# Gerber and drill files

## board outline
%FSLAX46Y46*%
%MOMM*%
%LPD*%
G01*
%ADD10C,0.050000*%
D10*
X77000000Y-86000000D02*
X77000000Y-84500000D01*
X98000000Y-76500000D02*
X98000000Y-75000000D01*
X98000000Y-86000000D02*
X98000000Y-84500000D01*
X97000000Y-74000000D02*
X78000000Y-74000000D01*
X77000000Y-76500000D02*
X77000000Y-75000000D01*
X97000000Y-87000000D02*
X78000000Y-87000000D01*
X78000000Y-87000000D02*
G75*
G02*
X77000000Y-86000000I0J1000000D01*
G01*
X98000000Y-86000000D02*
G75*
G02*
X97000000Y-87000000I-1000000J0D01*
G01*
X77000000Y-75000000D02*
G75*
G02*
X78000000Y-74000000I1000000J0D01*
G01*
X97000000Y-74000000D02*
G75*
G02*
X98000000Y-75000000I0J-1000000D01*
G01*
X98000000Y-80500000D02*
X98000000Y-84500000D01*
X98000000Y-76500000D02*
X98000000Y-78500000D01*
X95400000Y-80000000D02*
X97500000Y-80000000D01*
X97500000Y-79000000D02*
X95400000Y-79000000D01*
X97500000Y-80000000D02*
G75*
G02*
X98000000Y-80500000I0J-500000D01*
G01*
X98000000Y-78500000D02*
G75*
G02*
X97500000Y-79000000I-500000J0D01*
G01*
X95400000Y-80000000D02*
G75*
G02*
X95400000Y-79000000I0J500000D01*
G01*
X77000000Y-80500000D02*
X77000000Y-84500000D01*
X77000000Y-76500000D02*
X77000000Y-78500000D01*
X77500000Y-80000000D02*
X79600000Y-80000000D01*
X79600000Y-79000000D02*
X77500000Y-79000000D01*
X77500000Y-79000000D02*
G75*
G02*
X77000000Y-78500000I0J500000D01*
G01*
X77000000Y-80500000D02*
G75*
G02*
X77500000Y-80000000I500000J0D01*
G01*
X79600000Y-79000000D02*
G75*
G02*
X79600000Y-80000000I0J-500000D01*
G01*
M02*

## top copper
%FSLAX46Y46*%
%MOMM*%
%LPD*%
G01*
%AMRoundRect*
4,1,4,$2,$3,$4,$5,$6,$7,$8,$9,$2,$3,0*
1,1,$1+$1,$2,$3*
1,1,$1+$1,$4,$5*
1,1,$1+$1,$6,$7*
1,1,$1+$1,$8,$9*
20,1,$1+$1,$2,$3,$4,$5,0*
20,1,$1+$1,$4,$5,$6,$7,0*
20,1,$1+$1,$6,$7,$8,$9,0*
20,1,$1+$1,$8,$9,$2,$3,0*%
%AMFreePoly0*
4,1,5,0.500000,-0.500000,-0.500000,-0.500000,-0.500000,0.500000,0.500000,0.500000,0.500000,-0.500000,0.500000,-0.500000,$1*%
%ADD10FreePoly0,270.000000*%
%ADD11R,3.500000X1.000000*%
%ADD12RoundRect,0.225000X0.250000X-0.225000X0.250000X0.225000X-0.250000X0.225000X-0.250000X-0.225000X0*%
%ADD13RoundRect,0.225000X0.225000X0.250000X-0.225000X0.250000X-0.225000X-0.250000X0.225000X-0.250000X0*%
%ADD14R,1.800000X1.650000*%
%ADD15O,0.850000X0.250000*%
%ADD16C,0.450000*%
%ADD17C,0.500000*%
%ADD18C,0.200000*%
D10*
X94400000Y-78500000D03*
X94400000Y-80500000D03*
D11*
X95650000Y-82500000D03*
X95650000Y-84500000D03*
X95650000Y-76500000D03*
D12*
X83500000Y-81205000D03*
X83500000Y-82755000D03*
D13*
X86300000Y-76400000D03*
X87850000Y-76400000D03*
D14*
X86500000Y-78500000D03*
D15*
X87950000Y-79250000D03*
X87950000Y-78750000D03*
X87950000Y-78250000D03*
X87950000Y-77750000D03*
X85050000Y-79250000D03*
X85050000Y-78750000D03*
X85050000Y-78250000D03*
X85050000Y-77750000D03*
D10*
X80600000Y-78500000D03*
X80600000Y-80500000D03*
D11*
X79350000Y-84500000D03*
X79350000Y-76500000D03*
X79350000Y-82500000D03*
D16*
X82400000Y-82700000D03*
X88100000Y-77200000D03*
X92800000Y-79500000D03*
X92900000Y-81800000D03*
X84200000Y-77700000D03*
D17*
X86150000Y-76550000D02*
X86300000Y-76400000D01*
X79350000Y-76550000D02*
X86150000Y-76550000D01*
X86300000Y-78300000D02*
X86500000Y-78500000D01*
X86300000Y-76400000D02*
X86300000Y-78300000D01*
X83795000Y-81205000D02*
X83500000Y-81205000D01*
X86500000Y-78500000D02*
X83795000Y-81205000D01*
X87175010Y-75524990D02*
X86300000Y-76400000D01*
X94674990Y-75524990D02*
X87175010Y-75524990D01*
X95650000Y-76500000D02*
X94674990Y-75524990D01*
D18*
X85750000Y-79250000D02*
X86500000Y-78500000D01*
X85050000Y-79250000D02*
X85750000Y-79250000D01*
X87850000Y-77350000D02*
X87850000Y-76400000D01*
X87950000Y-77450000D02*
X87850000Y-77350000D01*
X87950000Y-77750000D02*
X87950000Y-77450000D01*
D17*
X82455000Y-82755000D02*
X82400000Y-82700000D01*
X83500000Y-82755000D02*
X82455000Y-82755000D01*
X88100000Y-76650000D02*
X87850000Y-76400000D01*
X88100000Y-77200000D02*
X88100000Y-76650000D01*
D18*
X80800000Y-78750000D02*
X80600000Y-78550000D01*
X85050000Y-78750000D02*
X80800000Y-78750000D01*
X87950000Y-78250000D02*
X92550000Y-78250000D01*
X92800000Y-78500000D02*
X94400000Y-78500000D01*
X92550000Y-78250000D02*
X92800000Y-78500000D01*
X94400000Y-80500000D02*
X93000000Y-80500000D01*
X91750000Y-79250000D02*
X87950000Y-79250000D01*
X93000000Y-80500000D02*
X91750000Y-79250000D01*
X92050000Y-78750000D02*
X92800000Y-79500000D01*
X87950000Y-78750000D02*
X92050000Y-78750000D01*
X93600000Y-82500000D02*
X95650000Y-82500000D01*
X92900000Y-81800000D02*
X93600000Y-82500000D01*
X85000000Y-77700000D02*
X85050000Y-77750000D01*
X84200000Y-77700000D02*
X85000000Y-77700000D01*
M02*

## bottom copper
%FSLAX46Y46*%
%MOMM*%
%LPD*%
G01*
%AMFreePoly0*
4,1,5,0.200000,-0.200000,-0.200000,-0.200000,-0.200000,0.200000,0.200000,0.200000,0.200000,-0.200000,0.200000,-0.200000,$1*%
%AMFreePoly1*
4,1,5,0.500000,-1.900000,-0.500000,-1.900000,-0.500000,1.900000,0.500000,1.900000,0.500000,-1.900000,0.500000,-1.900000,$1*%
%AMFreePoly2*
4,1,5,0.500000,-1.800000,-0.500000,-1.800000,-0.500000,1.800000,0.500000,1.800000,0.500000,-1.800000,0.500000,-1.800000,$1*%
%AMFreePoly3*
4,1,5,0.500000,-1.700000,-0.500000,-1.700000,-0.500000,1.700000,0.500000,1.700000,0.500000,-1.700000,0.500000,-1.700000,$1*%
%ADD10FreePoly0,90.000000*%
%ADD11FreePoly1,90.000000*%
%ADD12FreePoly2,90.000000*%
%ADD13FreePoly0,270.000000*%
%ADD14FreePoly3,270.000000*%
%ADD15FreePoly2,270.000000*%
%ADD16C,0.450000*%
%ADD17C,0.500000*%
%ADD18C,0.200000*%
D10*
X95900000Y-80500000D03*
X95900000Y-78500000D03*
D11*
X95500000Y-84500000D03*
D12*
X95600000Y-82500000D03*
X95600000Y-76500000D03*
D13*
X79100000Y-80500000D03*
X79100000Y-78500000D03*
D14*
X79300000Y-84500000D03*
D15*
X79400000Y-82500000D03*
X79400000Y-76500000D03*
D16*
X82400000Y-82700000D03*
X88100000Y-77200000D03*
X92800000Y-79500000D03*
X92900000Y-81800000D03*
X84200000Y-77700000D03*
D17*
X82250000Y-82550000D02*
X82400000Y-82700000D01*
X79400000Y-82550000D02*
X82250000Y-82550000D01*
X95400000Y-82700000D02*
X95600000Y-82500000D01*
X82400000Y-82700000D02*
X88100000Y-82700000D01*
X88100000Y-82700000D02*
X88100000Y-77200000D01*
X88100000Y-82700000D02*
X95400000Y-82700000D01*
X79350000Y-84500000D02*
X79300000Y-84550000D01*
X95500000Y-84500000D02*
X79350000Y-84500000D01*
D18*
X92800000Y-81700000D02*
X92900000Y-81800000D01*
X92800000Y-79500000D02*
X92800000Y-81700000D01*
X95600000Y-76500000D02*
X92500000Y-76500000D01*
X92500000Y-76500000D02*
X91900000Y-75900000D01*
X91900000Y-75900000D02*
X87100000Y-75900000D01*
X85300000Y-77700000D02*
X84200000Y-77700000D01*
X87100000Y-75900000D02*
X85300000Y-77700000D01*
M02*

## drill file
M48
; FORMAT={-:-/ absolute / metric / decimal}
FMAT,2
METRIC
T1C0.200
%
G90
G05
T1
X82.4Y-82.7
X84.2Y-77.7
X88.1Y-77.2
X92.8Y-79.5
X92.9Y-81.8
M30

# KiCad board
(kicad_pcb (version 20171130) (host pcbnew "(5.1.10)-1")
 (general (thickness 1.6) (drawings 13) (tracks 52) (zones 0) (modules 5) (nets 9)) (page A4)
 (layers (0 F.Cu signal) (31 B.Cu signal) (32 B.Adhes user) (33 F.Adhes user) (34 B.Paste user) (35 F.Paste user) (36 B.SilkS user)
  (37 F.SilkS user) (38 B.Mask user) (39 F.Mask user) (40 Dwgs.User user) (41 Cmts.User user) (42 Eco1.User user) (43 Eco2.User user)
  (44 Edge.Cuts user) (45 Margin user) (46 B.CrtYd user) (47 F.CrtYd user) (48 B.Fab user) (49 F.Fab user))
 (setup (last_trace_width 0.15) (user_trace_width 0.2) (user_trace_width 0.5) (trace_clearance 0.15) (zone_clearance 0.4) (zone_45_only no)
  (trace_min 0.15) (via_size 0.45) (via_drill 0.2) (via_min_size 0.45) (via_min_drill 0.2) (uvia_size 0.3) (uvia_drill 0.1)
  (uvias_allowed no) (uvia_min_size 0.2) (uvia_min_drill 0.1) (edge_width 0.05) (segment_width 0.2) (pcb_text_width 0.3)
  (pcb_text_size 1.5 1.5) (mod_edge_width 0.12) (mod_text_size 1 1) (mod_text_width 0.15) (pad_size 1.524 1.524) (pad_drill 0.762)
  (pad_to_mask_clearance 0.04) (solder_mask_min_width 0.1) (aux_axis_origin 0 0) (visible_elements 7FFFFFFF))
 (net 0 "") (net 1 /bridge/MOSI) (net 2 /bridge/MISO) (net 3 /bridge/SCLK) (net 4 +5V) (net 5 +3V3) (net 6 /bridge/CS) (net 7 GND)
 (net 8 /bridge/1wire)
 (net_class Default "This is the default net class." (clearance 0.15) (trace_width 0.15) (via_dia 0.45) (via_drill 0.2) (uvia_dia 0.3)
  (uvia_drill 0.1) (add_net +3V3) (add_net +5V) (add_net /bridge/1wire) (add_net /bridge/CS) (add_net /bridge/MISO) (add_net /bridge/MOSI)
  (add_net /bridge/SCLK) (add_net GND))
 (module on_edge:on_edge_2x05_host (layer F.Cu) (at 98 80.5 270)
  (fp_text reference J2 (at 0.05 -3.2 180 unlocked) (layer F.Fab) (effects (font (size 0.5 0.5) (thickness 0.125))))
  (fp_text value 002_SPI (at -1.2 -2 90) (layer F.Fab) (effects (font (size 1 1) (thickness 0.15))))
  (fp_line (start 0 0) (end 4 0) (layer Edge.Cuts) (width 0.05))
  (fp_line (start -4 0) (end -2 0) (layer Edge.Cuts) (width 0.05))
  (fp_line (start -0.5 2.6) (end -0.5 0.5) (layer Edge.Cuts) (width 0.05))
  (fp_line (start -1.5 0.5) (end -1.5 2.6) (layer Edge.Cuts) (width 0.05))
  (fp_arc (start 0 0.5) (end 0 0) (angle -90) (layer Edge.Cuts) (width 0.05))
  (fp_arc (start -2 0.5) (end -1.5 0.5) (angle -90) (layer Edge.Cuts) (width 0.05))
  (fp_arc (start -1 2.6) (end -1.5 2.6) (angle -180) (layer Edge.Cuts) (width 0.05))
  (pad 2 smd custom (at -2 3.6 270) (size 1 1) (layers F.Cu F.Mask) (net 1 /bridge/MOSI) (zone_connect 0)
   (options (clearance outline) (anchor rect)) (primitives))
  (pad 3 smd custom (at 0 3.6 270) (size 1 1) (layers F.Cu F.Mask) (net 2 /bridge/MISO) (zone_connect 0)
   (options (clearance outline) (anchor rect)) (primitives))
  (pad 8 smd custom (at 0 2.1 90) (size 0.4 0.4) (layers B.Cu B.Mask) (zone_connect 0) (options (clearance outline) (anchor rect))
   (primitives))
  (pad 7 smd custom (at -2 2.1 90) (size 0.4 0.4) (layers B.Cu B.Mask) (zone_connect 0) (options (clearance outline) (anchor rect))
   (primitives))
  (pad 4 smd rect (at 2 2.35 270) (size 1 3.5) (layers F.Cu F.Mask) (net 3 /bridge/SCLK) (zone_connect 0))
  (pad 10 smd custom (at 4 2.5 90) (size 1 3.8) (layers B.Cu B.Mask) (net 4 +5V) (zone_connect 0)
   (options (clearance outline) (anchor rect)) (primitives))
  (pad 9 smd custom (at 2 2.4 90) (size 1 3.6) (layers B.Cu B.Mask) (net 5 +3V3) (zone_connect 0)
   (options (clearance outline) (anchor rect)) (primitives))
  (pad 6 smd custom (at -4 2.4 90) (size 1 3.6) (layers B.Cu B.Mask) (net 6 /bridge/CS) (zone_connect 0)
   (options (clearance outline) (anchor rect)) (primitives))
  (pad 5 smd rect (at 4 2.35 270) (size 1 3.5) (layers F.Cu F.Mask) (zone_connect 0))
  (pad 1 smd rect (at -4 2.35 270) (size 1 3.5) (layers F.Cu F.Mask) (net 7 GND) (zone_connect 0)))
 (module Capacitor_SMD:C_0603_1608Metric (layer F.Cu) (at 83.5 81.98 90)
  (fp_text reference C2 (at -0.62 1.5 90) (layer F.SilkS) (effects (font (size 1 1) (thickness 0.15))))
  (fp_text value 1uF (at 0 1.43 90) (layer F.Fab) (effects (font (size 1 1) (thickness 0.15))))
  (pad 2 smd roundrect (at 0.775 0 90) (size 0.9 0.95) (layers F.Cu F.Paste F.Mask) (roundrect_rratio 0.25) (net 7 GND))
  (pad 1 smd roundrect (at -0.775 0 90) (size 0.9 0.95) (layers F.Cu F.Paste F.Mask) (roundrect_rratio 0.25) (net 5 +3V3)))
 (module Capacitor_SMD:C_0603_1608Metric (layer F.Cu) (at 87.075 76.4 180)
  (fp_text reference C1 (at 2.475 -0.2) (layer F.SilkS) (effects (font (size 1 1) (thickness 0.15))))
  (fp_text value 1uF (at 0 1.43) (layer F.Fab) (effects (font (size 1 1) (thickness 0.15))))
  (pad 2 smd roundrect (at 0.775 0 180) (size 0.9 0.95) (layers F.Cu F.Paste F.Mask) (roundrect_rratio 0.25) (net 7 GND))
  (pad 1 smd roundrect (at -0.775 0 180) (size 0.9 0.95) (layers F.Cu F.Paste F.Mask) (roundrect_rratio 0.25) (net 5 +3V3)))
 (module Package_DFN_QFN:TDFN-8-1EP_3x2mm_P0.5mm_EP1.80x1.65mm (layer F.Cu) (at 86.5 78.5)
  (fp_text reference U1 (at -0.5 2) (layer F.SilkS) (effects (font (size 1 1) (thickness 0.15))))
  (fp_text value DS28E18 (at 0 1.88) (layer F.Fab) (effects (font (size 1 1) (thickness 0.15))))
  (pad "" smd rect (at 0 0.5) (size 0.7 0.65) (layers F.Paste))
  (pad "" smd rect (at 0 -0.5) (size 0.7 0.65) (layers F.Paste)) (pad "" smd rect (at 0 0) (size 1.8 0.7) (layers F.Paste))
  (pad 9 smd rect (at 0 0) (size 1.8 1.65) (layers F.Cu F.Mask) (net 7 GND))
  (pad 5 smd oval (at 1.45 0.75) (size 0.85 0.25) (layers F.Cu F.Paste F.Mask) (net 2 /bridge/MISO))
  (pad 6 smd oval (at 1.45 0.25) (size 0.85 0.25) (layers F.Cu F.Paste F.Mask) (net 3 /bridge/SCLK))
  (pad 7 smd oval (at 1.45 -0.25) (size 0.85 0.25) (layers F.Cu F.Paste F.Mask) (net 1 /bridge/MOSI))
  (pad 8 smd oval (at 1.45 -0.75) (size 0.85 0.25) (layers F.Cu F.Paste F.Mask) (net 5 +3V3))
  (pad 4 smd oval (at -1.45 0.75) (size 0.85 0.25) (layers F.Cu F.Paste F.Mask) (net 7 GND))
  (pad 3 smd oval (at -1.45 0.25) (size 0.85 0.25) (layers F.Cu F.Paste F.Mask) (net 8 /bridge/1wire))
  (pad 2 smd oval (at -1.45 -0.25) (size 0.85 0.25) (layers F.Cu F.Paste F.Mask))
  (pad 1 smd oval (at -1.45 -0.75) (size 0.85 0.25) (layers F.Cu F.Paste F.Mask) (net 6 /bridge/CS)))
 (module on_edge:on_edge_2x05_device (layer F.Cu) (at 77 80.5 270)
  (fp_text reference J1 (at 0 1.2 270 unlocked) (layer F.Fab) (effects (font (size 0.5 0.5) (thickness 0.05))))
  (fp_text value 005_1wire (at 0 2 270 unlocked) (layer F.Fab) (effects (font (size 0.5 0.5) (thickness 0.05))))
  (fp_line (start 0 0) (end 4 0) (layer Edge.Cuts) (width 0.05))
  (fp_line (start -4 0) (end -2 0) (layer Edge.Cuts) (width 0.05))
  (fp_line (start -0.5 -0.5) (end -0.5 -2.6) (layer Edge.Cuts) (width 0.05))
  (fp_line (start -1.5 -2.6) (end -1.5 -0.5) (layer Edge.Cuts) (width 0.05))
  (fp_arc (start -2 -0.5) (end -2 0) (angle -90) (layer Edge.Cuts) (width 0.05))
  (fp_arc (start 0 -0.5) (end -0.5 -0.5) (angle -90) (layer Edge.Cuts) (width 0.05))
  (fp_arc (start -1 -2.6) (end -0.5 -2.6) (angle -180) (layer Edge.Cuts) (width 0.05))
  (pad 2 smd custom (at -2 -3.6 270) (size 1 1) (layers F.Cu F.Mask) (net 8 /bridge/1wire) (zone_connect 0)
   (options (clearance outline) (anchor rect)) (primitives))
  (pad 3 smd custom (at 0 -3.6 270) (size 1 1) (layers F.Cu F.Mask) (zone_connect 0) (options (clearance outline) (anchor rect))
   (primitives))
  (pad 8 smd custom (at 0 -2.1 270) (size 0.4 0.4) (layers B.Cu B.Mask) (zone_connect 0) (options (clearance outline) (anchor rect))
   (primitives))
  (pad 7 smd custom (at -2 -2.1 270) (size 0.4 0.4) (layers B.Cu B.Mask) (zone_connect 0) (options (clearance outline) (anchor rect))
   (primitives))
  (pad 10 smd custom (at 4 -2.3 270) (size 1 3.4) (layers B.Cu B.Mask) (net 4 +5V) (zone_connect 0)
   (options (clearance outline) (anchor rect)) (primitives))
  (pad 9 smd custom (at 2 -2.4 270) (size 1 3.6) (layers B.Cu B.Mask) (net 5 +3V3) (zone_connect 0)
   (options (clearance outline) (anchor rect)) (primitives))
  (pad 6 smd custom (at -4 -2.4 270) (size 1 3.6) (layers B.Cu B.Mask) (zone_connect 0) (options (clearance outline) (anchor rect))
   (primitives))
  (pad 5 smd rect (at 4 -2.35 90) (size 1 3.5) (layers F.Cu F.Mask) (zone_connect 0))
  (pad 1 smd rect (at -4 -2.35 90) (size 1 3.5) (layers F.Cu F.Mask) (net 7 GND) (zone_connect 0))
  (pad 4 smd rect (at 2 -2.35 90) (size 1 3.5) (layers F.Cu F.Mask) (zone_connect 0)))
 (gr_line (start 77 86) (end 77 84.5) (layer Edge.Cuts) (width 0.05))
 (gr_line (start 98 76.5) (end 98 75) (layer Edge.Cuts) (width 0.05))
 (gr_line (start 98 86) (end 98 84.5) (layer Edge.Cuts) (width 0.05))
 (gr_line (start 97 74) (end 78 74) (layer Edge.Cuts) (width 0.05))
 (gr_line (start 77 76.5) (end 77 75) (layer Edge.Cuts) (width 0.05))
 (gr_line (start 97 87) (end 78 87) (layer Edge.Cuts) (width 0.05))
 (gr_arc (start 78 86) (end 77 86) (angle -90) (layer Edge.Cuts) (width 0.05))
 (gr_arc (start 97 86) (end 97 87) (angle -90) (layer Edge.Cuts) (width 0.05))
 (gr_arc (start 78 75) (end 78 74) (angle -90) (layer Edge.Cuts) (width 0.05))
 (gr_arc (start 97 75) (end 98 75) (angle -90) (layer Edge.Cuts) (width 0.05))
 (segment (start 86.15 76.55) (end 86.3 76.4) (width 0.5) (layer F.Cu) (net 7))
 (segment (start 79.35 76.55) (end 86.15 76.55) (width 0.5) (layer F.Cu) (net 7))
 (segment (start 86.3 78.3) (end 86.5 78.5) (width 0.5) (layer F.Cu) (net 7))
 (segment (start 86.3 76.4) (end 86.3 78.3) (width 0.5) (layer F.Cu) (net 7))
 (segment (start 83.795 81.205) (end 83.5 81.205) (width 0.5) (layer F.Cu) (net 7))
 (segment (start 86.5 78.5) (end 83.795 81.205) (width 0.5) (layer F.Cu) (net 7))
 (segment (start 87.17501 75.52499) (end 86.3 76.4) (width 0.5) (layer F.Cu) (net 7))
 (segment (start 94.67499 75.52499) (end 87.17501 75.52499) (width 0.5) (layer F.Cu) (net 7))
 (segment (start 95.65 76.5) (end 94.67499 75.52499) (width 0.5) (layer F.Cu) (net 7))
 (segment (start 85.75 79.25) (end 86.5 78.5) (width 0.2) (layer F.Cu) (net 7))
 (segment (start 85.05 79.25) (end 85.75 79.25) (width 0.2) (layer F.Cu) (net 7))
 (segment (start 82.25 82.55) (end 82.4 82.7) (width 0.5) (layer B.Cu) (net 5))
 (via (at 82.4 82.7) (size 0.45) (drill 0.2) (layers F.Cu B.Cu) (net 5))
 (segment (start 79.4 82.55) (end 82.25 82.55) (width 0.5) (layer B.Cu) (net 5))
 (segment (start 87.85 77.35) (end 87.85 76.4) (width 0.2) (layer F.Cu) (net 5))
 (segment (start 87.95 77.45) (end 87.85 77.35) (width 0.2) (layer F.Cu) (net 5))
 (segment (start 87.95 77.75) (end 87.95 77.45) (width 0.2) (layer F.Cu) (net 5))
 (segment (start 82.455 82.755) (end 82.4 82.7) (width 0.5) (layer F.Cu) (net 5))
 (segment (start 83.5 82.755) (end 82.455 82.755) (width 0.5) (layer F.Cu) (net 5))
 (segment (start 95.4 82.7) (end 95.6 82.5) (width 0.5) (layer B.Cu) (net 5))
 (via (at 88.1 77.2) (size 0.45) (drill 0.2) (layers F.Cu B.Cu) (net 5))
 (segment (start 82.4 82.7) (end 88.1 82.7) (width 0.5) (layer B.Cu) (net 5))
 (segment (start 88.1 82.7) (end 88.1 77.2) (width 0.5) (layer B.Cu) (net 5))
 (segment (start 88.1 82.7) (end 95.4 82.7) (width 0.5) (layer B.Cu) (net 5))
 (segment (start 88.1 76.65) (end 87.85 76.4) (width 0.5) (layer F.Cu) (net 5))
 (segment (start 88.1 77.2) (end 88.1 76.65) (width 0.5) (layer F.Cu) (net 5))
 (segment (start 80.8 78.75) (end 80.6 78.55) (width 0.2) (layer F.Cu) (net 8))
 (segment (start 85.05 78.75) (end 80.8 78.75) (width 0.2) (layer F.Cu) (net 8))
 (segment (start 79.35 84.5) (end 79.3 84.55) (width 0.5) (layer B.Cu) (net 4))
 (segment (start 95.5 84.5) (end 79.35 84.5) (width 0.5) (layer B.Cu) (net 4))
 (segment (start 87.95 78.25) (end 92.55 78.25) (width 0.2) (layer F.Cu) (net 1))
 (segment (start 92.8 78.5) (end 94.4 78.5) (width 0.2) (layer F.Cu) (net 1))
 (segment (start 92.55 78.25) (end 92.8 78.5) (width 0.2) (layer F.Cu) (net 1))
 (segment (start 94.4 80.5) (end 93 80.5) (width 0.2) (layer F.Cu) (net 2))
 (segment (start 91.75 79.25) (end 87.95 79.25) (width 0.2) (layer F.Cu) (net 2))
 (segment (start 93 80.5) (end 91.75 79.25) (width 0.2) (layer F.Cu) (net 2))
 (via (at 92.8 79.5) (size 0.45) (drill 0.2) (layers F.Cu B.Cu) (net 3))
 (segment (start 92.05 78.75) (end 92.8 79.5) (width 0.2) (layer F.Cu) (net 3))
 (segment (start 87.95 78.75) (end 92.05 78.75) (width 0.2) (layer F.Cu) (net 3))
 (via (at 92.9 81.8) (size 0.45) (drill 0.2) (layers F.Cu B.Cu) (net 3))
 (segment (start 92.8 81.7) (end 92.9 81.8) (width 0.2) (layer B.Cu) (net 3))
 (segment (start 92.8 79.5) (end 92.8 81.7) (width 0.2) (layer B.Cu) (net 3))
 (segment (start 93.6 82.5) (end 95.65 82.5) (width 0.2) (layer F.Cu) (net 3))
 (segment (start 92.9 81.8) (end 93.6 82.5) (width 0.2) (layer F.Cu) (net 3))
 (segment (start 95.6 76.5) (end 92.5 76.5) (width 0.2) (layer B.Cu) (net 6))
 (segment (start 92.5 76.5) (end 91.9 75.9) (width 0.2) (layer B.Cu) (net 6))
 (segment (start 91.9 75.9) (end 87.1 75.9) (width 0.2) (layer B.Cu) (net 6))
 (via (at 84.2 77.7) (size 0.45) (drill 0.2) (layers F.Cu B.Cu) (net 6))
 (segment (start 85.3 77.7) (end 84.2 77.7) (width 0.2) (layer B.Cu) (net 6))
 (segment (start 87.1 75.9) (end 85.3 77.7) (width 0.2) (layer B.Cu) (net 6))
 (segment (start 85 77.7) (end 85.05 77.75) (width 0.2) (layer F.Cu) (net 6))
 (segment (start 84.2 77.7) (end 85 77.7) (width 0.2) (layer F.Cu) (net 6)))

